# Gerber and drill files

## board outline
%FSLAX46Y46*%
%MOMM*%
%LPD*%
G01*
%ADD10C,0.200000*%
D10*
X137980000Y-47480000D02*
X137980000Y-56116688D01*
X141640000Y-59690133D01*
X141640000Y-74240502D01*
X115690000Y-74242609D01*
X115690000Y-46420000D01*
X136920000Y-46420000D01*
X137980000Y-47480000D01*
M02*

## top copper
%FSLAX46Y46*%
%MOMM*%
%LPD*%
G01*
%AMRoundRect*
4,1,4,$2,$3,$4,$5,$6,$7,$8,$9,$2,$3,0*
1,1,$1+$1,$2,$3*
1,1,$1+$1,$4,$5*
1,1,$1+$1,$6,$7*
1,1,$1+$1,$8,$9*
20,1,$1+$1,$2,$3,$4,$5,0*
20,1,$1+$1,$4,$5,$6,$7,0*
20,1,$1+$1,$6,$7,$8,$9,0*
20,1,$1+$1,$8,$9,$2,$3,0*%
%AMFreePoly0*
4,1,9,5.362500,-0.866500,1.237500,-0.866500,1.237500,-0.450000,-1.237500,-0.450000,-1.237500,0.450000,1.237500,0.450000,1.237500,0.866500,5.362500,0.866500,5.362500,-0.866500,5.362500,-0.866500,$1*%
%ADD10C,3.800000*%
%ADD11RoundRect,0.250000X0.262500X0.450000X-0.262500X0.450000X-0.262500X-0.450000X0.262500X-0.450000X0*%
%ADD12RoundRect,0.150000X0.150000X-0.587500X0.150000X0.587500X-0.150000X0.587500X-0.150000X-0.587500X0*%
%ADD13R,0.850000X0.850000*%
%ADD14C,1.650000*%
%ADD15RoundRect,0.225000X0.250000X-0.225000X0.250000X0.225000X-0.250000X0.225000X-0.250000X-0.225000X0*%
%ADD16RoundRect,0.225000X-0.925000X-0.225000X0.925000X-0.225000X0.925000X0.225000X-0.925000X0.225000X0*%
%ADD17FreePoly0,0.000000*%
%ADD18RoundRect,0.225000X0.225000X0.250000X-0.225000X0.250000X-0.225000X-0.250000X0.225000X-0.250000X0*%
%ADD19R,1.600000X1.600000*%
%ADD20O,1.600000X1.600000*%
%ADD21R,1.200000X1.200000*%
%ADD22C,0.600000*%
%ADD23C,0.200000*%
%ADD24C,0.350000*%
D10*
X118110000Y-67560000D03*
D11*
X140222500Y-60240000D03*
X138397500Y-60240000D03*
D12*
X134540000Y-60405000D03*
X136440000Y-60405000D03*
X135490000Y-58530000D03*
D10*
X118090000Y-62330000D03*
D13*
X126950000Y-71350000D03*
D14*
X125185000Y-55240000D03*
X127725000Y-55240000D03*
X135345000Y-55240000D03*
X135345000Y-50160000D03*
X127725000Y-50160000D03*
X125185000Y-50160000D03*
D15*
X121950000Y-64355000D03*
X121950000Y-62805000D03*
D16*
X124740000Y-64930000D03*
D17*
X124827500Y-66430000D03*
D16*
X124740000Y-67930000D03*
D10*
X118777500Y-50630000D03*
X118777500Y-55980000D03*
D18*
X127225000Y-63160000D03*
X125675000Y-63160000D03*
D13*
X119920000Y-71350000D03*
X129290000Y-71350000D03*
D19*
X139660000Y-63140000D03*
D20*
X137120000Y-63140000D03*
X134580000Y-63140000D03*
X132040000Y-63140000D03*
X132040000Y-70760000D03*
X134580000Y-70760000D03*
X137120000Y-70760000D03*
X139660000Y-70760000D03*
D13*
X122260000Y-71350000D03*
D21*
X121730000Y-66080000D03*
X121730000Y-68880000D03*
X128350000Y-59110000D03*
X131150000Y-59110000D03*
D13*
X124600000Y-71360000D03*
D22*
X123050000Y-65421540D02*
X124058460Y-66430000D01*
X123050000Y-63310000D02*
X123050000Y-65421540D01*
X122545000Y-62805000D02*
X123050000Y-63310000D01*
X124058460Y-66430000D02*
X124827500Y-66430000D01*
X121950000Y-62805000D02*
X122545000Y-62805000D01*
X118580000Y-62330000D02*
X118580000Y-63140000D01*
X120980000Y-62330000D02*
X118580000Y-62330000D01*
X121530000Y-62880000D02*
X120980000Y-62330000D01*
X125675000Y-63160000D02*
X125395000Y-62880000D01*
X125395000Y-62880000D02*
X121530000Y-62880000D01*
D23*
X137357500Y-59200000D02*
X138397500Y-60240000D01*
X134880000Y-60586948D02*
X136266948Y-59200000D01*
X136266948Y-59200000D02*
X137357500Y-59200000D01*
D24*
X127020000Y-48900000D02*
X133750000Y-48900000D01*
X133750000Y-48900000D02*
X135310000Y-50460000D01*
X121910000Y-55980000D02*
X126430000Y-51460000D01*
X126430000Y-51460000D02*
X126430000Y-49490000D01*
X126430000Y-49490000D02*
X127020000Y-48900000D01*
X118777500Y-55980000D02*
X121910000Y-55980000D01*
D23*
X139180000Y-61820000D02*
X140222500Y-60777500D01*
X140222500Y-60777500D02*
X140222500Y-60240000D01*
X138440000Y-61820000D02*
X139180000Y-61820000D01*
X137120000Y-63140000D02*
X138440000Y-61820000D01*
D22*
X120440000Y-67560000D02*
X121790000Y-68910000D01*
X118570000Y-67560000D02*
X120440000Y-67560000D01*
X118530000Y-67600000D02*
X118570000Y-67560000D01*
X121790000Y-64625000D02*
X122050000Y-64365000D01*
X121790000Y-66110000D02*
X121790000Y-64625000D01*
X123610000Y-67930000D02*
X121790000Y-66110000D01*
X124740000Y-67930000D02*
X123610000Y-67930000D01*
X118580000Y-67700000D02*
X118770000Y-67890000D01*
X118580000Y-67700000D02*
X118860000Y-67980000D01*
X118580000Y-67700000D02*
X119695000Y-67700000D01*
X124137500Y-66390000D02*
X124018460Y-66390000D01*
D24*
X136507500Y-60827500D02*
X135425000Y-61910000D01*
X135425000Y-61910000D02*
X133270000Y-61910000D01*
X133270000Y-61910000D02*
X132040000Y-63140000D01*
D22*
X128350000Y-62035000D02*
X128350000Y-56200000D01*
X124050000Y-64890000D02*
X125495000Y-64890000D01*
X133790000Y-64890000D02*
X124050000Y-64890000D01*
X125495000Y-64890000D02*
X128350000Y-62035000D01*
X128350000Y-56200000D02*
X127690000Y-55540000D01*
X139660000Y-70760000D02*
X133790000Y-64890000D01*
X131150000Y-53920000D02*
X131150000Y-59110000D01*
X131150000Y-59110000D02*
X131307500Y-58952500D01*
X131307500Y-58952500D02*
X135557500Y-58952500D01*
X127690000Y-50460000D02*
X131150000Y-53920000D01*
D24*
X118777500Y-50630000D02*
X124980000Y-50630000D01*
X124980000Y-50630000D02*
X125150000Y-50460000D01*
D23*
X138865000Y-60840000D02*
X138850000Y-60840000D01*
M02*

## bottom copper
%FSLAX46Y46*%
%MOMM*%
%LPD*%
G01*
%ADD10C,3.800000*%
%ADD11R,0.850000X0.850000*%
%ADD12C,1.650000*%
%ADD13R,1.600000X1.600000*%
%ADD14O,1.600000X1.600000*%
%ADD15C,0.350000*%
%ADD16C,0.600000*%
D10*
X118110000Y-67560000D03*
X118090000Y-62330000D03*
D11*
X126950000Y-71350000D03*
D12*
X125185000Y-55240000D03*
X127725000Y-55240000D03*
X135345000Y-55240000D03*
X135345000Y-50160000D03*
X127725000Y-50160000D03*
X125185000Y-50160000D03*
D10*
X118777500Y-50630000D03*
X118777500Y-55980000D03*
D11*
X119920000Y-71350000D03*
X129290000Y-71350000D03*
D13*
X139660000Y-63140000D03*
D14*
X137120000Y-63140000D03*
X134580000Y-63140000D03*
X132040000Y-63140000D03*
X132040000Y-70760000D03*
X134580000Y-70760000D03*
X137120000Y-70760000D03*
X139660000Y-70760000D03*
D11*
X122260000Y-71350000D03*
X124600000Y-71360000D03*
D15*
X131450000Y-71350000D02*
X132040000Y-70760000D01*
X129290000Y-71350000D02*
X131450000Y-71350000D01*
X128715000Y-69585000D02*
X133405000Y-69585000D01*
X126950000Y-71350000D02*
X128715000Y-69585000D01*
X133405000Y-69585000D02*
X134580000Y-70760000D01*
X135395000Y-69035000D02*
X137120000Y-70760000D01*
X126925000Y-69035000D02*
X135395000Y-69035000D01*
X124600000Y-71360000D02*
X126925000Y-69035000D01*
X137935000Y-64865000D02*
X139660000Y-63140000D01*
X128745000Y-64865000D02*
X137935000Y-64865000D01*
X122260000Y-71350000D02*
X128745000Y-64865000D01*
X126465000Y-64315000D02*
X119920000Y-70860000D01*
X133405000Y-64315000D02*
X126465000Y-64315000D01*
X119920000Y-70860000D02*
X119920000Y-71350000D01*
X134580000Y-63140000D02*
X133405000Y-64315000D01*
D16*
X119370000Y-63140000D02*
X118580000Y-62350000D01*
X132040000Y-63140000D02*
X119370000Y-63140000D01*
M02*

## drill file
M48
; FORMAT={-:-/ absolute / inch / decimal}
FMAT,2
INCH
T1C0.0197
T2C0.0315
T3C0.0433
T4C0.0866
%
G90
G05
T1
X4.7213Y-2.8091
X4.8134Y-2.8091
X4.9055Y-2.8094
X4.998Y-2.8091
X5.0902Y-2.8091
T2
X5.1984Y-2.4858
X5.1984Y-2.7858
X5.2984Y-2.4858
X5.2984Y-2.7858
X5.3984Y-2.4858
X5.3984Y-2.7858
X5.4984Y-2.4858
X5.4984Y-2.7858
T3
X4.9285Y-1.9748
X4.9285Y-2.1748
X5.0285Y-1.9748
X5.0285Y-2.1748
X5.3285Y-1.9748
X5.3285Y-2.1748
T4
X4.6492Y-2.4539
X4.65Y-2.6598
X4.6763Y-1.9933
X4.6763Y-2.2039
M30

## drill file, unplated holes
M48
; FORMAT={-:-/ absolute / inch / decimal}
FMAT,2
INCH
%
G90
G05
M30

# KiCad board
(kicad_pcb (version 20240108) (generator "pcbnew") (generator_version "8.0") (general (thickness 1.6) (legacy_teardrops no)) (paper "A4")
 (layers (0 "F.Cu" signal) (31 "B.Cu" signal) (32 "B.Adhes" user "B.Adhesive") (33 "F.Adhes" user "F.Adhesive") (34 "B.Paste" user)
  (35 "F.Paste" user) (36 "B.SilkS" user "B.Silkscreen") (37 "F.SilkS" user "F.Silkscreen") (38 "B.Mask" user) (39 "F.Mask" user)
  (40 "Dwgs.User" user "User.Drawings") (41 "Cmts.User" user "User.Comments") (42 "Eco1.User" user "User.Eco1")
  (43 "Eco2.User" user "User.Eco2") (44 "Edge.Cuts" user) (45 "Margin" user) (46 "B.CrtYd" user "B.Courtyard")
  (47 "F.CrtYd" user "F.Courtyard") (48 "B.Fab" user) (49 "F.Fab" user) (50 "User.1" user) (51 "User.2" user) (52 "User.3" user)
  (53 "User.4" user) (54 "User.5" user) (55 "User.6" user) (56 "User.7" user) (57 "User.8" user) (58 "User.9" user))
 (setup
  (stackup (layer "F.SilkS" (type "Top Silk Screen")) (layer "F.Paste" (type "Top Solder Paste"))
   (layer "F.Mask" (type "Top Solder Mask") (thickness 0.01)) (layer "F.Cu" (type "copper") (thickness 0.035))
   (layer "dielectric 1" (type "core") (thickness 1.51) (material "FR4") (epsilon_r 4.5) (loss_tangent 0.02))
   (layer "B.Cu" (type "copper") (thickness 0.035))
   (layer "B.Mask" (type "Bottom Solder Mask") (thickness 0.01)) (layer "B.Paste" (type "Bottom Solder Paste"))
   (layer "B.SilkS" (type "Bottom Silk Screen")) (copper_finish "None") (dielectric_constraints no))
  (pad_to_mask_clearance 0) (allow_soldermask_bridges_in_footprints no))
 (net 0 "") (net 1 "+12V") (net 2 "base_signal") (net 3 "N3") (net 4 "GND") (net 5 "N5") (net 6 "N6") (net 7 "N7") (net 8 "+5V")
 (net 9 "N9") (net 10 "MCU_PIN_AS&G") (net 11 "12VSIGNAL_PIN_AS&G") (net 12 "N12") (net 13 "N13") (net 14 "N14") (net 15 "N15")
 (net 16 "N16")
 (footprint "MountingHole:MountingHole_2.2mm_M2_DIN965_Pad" (layer "F.Cu") (at 118.11 67.56)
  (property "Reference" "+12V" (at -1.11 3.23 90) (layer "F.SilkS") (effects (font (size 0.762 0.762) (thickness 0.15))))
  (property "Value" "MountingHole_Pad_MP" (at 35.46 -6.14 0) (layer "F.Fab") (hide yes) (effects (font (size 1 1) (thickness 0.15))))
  (pad "1" thru_hole circle (at 0 0) (size 3.8 3.8) (drill 2.2) (layers "*.Cu" "*.Mask") (remove_unused_layers no) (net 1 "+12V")))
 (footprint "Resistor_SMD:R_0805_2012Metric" (layer "F.Cu") (at 139.31 60.24 180)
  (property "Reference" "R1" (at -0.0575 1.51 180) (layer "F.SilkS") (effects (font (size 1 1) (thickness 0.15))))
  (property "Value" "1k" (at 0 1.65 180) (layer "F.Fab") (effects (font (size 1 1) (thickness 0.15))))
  (pad "1" smd roundrect (at -0.9125 0 180) (size 1.025 1.4) (layers "F.Cu" "F.Paste" "F.Mask") (roundrect_rratio 0.243902)
   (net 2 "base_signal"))
  (pad "2" smd roundrect (at 0.9125 0 180) (size 1.025 1.4) (layers "F.Cu" "F.Paste" "F.Mask") (roundrect_rratio 0.243902) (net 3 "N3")))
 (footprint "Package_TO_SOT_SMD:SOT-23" (layer "F.Cu") (at 135.49 59.4675 90)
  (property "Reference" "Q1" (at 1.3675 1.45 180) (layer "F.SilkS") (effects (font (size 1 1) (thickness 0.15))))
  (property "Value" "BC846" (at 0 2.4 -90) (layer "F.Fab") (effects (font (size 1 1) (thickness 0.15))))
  (pad "1" smd roundrect (at -0.9375 -0.95 90) (size 1.475 0.6) (layers "F.Cu" "F.Paste" "F.Mask") (roundrect_rratio 0.25) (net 3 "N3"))
  (pad "2" smd roundrect (at -0.9375 0.95 90) (size 1.475 0.6) (layers "F.Cu" "F.Paste" "F.Mask") (roundrect_rratio 0.25) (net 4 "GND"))
  (pad "3" smd roundrect (at 0.9375 0 90) (size 1.475 0.6) (layers "F.Cu" "F.Paste" "F.Mask") (roundrect_rratio 0.25) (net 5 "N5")))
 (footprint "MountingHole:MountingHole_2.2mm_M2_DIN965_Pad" (layer "F.Cu") (at 118.09 62.33)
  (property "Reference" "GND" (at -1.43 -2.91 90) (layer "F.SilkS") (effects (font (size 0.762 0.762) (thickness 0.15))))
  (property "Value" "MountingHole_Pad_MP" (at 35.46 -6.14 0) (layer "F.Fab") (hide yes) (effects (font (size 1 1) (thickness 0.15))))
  (pad "1" thru_hole circle (at 0 0) (size 3.8 3.8) (drill 2.2) (layers "*.Cu" "*.Mask") (remove_unused_layers no) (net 4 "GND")))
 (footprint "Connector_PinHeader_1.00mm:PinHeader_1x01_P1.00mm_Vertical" (layer "F.Cu") (at 126.95 71.35)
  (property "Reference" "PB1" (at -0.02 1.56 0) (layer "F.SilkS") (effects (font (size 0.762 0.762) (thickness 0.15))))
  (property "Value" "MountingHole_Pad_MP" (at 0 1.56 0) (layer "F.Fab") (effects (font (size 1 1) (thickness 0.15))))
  (pad "1" thru_hole rect (at 0 0) (size 0.85 0.85) (drill 0.5) (layers "*.Cu" "*.Mask") (remove_unused_layers no) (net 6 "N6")))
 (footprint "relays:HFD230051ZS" (layer "F.Cu") (at 125.185 55.24)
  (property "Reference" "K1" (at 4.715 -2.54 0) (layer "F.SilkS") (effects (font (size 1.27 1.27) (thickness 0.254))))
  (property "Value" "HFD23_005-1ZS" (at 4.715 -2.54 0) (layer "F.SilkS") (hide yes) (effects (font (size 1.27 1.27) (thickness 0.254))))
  (pad "1" thru_hole circle (at 0 0) (size 1.65 1.65) (drill 1.1) (layers "*.Cu" "*.Mask") (remove_unused_layers no) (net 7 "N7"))
  (pad "2" thru_hole circle (at 2.54 0) (size 1.65 1.65) (drill 1.1) (layers "*.Cu" "*.Mask") (remove_unused_layers no) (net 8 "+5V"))
  (pad "3" thru_hole circle (at 10.16 0) (size 1.65 1.65) (drill 1.1) (layers "*.Cu" "*.Mask") (remove_unused_layers no) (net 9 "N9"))
  (pad "4" thru_hole circle (at 10.16 -5.08) (size 1.65 1.65) (drill 1.1) (layers "*.Cu" "*.Mask") (remove_unused_layers no)
   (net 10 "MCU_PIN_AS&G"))
  (pad "5" thru_hole circle (at 2.54 -5.08) (size 1.65 1.65) (drill 1.1) (layers "*.Cu" "*.Mask") (remove_unused_layers no) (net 5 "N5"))
  (pad "6" thru_hole circle (at 0 -5.08) (size 1.65 1.65) (drill 1.1) (layers "*.Cu" "*.Mask") (remove_unused_layers no)
   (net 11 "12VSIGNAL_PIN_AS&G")))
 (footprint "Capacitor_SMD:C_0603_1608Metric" (layer "F.Cu") (at 121.95 63.58 90)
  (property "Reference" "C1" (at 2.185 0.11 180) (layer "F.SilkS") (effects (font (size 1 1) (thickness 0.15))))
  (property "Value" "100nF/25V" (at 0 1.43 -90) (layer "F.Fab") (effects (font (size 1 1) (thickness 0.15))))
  (pad "1" smd roundrect (at -0.775 0 90) (size 0.9 0.95) (layers "F.Cu" "F.Paste" "F.Mask") (roundrect_rratio 0.25) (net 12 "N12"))
  (pad "2" smd roundrect (at 0.775 0 90) (size 0.9 0.95) (layers "F.Cu" "F.Paste" "F.Mask") (roundrect_rratio 0.25) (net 4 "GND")))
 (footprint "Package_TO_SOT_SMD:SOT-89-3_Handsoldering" (layer "F.Cu") (at 127.19 66.43)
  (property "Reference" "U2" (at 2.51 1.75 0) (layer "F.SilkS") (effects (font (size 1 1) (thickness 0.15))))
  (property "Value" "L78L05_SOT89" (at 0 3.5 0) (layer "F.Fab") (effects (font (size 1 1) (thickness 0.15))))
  (pad "1" smd roundrect (at -2.45 -1.5) (size 2.3 0.9) (layers "F.Cu" "F.Paste" "F.Mask") (roundrect_rratio 0.25) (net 8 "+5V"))
  (pad "2" smd custom (at -2.3625 0) (size 2.475 0.9) (layers "F.Cu" "F.Paste" "F.Mask") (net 4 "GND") (zone_connect 2)
   (thermal_bridge_angle 45) (options (clearance outline) (anchor rect)) (primitives))
  (pad "3" smd roundrect (at -2.45 1.5) (size 2.3 0.9) (layers "F.Cu" "F.Paste" "F.Mask") (roundrect_rratio 0.25) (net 12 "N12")))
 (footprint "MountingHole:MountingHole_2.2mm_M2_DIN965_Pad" (layer "F.Cu") (at 118.7775 50.63)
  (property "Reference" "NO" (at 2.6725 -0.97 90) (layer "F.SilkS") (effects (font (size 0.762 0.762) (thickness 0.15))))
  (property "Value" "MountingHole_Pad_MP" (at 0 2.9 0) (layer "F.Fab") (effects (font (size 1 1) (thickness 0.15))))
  (pad "1" thru_hole circle (at 0 0) (size 3.8 3.8) (drill 2.2) (layers "*.Cu" "*.Mask") (remove_unused_layers no)
   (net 11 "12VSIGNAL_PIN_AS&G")))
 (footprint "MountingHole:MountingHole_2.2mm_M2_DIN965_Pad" (layer "F.Cu") (at 118.7775 55.98)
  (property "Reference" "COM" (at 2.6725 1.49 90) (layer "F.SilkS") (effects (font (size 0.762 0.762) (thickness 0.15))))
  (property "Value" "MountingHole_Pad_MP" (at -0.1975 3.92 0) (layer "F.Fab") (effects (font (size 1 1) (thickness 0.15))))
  (pad "1" thru_hole circle (at 0 0) (size 3.8 3.8) (drill 2.2) (layers "*.Cu" "*.Mask") (remove_unused_layers no) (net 10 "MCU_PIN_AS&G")))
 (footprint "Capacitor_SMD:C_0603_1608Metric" (layer "F.Cu") (at 126.45 63.16 180)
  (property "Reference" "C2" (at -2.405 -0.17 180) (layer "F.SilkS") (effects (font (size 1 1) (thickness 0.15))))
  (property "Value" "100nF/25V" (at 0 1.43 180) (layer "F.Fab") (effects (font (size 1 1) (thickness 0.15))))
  (pad "1" smd roundrect (at -0.775 0 180) (size 0.9 0.95) (layers "F.Cu" "F.Paste" "F.Mask") (roundrect_rratio 0.25) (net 8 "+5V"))
  (pad "2" smd roundrect (at 0.775 0 180) (size 0.9 0.95) (layers "F.Cu" "F.Paste" "F.Mask") (roundrect_rratio 0.25) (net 4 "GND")))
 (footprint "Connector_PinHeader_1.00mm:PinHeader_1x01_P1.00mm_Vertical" (layer "F.Cu") (at 119.92 71.35)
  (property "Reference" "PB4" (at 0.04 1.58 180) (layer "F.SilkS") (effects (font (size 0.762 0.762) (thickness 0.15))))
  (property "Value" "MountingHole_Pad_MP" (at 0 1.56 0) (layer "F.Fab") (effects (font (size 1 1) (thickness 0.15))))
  (pad "1" thru_hole rect (at 0 0) (size 0.85 0.85) (drill 0.5) (layers "*.Cu" "*.Mask") (remove_unused_layers no) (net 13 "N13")))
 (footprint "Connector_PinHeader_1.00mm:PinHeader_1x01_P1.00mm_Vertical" (layer "F.Cu") (at 129.29 71.35)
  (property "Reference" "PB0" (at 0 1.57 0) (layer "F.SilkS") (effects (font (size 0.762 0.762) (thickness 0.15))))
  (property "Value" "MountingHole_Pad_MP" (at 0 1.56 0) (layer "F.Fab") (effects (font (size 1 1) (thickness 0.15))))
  (pad "1" thru_hole rect (at 0 0) (size 0.85 0.85) (drill 0.5) (layers "*.Cu" "*.Mask") (remove_unused_layers no) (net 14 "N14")))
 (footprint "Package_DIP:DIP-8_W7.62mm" (layer "F.Cu") (at 139.66 63.14 -90)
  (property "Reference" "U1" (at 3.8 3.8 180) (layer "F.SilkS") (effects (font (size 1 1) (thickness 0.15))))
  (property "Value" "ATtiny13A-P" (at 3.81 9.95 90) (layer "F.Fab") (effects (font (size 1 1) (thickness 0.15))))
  (pad "1" thru_hole rect (at 0 0 270) (size 1.6 1.6) (drill 0.8) (layers "*.Cu" "*.Mask") (remove_unused_layers no) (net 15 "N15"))
  (pad "2" thru_hole oval (at 0 2.54 270) (size 1.6 1.6) (drill 0.8) (layers "*.Cu" "*.Mask") (remove_unused_layers no)
   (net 2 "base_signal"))
  (pad "3" thru_hole oval (at 0 5.08 270) (size 1.6 1.6) (drill 0.8) (layers "*.Cu" "*.Mask") (remove_unused_layers no) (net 13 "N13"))
  (pad "4" thru_hole oval (at 0 7.62 270) (size 1.6 1.6) (drill 0.8) (layers "*.Cu" "*.Mask") (remove_unused_layers no) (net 4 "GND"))
  (pad "5" thru_hole oval (at 7.62 7.62 270) (size 1.6 1.6) (drill 0.8) (layers "*.Cu" "*.Mask") (remove_unused_layers no) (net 14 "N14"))
  (pad "6" thru_hole oval (at 7.62 5.08 270) (size 1.6 1.6) (drill 0.8) (layers "*.Cu" "*.Mask") (remove_unused_layers no) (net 6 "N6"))
  (pad "7" thru_hole oval (at 7.62 2.54 270) (size 1.6 1.6) (drill 0.8) (layers "*.Cu" "*.Mask") (remove_unused_layers no) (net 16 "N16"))
  (pad "8" thru_hole oval (at 7.62 0 270) (size 1.6 1.6) (drill 0.8) (layers "*.Cu" "*.Mask") (remove_unused_layers no) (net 8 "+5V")))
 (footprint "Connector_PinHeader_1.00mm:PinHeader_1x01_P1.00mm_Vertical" (layer "F.Cu") (at 122.26 71.35)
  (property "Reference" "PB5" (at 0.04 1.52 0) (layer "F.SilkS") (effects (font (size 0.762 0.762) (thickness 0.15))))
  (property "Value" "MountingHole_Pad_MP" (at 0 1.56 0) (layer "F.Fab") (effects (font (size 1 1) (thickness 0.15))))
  (pad "1" thru_hole rect (at 0 0) (size 0.85 0.85) (drill 0.5) (layers "*.Cu" "*.Mask") (remove_unused_layers no) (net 15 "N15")))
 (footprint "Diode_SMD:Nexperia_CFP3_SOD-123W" (layer "F.Cu") (at 121.73 67.48 -90)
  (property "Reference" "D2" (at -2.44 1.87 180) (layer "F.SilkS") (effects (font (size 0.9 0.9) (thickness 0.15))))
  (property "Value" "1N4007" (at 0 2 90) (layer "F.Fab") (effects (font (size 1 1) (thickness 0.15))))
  (pad "1" smd rect (at -1.4 0 270) (size 1.2 1.2) (layers "F.Cu" "F.Paste" "F.Mask") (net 12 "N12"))
  (pad "2" smd rect (at 1.4 0 270) (size 1.2 1.2) (layers "F.Cu" "F.Paste" "F.Mask") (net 1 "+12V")))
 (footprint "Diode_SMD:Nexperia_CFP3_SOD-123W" (layer "F.Cu") (at 129.75 59.11)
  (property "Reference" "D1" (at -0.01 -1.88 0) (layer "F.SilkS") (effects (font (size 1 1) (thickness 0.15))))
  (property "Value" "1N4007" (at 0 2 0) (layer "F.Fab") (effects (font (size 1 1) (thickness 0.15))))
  (pad "1" smd rect (at -1.4 0) (size 1.2 1.2) (layers "F.Cu" "F.Paste" "F.Mask") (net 8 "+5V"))
  (pad "2" smd rect (at 1.4 0) (size 1.2 1.2) (layers "F.Cu" "F.Paste" "F.Mask") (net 5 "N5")))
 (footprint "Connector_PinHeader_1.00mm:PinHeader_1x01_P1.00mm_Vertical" (layer "F.Cu") (at 124.6 71.36)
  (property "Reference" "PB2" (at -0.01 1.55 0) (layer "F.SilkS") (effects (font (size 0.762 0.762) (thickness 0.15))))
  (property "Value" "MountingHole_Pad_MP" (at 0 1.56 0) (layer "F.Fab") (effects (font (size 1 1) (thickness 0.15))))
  (pad "1" thru_hole rect (at 0 0) (size 0.85 0.85) (drill 0.5) (layers "*.Cu" "*.Mask") (remove_unused_layers no) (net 16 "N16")))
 (gr_poly
  (pts (xy 115.69 74.242609) (xy 141.64 74.240502) (xy 141.64 59.690133) (xy 137.98 56.116688) (xy 137.98 47.48) (xy 136.92 46.42)
   (xy 115.69 46.42))
  (stroke (width 0.2) (type solid)) (fill none) (layer "Edge.Cuts"))
 (segment (start 118.58 67.7) (end 118.77 67.89) (width 0.6) (layer "F.Cu") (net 1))
 (segment (start 118.57 67.56) (end 120.44 67.56) (width 0.6) (layer "F.Cu") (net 1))
 (segment (start 118.53 67.6) (end 118.57 67.56) (width 0.6) (layer "F.Cu") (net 1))
 (segment (start 120.44 67.56) (end 121.79 68.91) (width 0.6) (layer "F.Cu") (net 1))
 (segment (start 118.58 67.7) (end 118.86 67.98) (width 0.6) (layer "F.Cu") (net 1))
 (segment (start 118.58 67.7) (end 119.695 67.7) (width 0.6) (layer "F.Cu") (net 1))
 (segment (start 125.395 62.88) (end 121.53 62.88) (width 0.6) (layer "F.Cu") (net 4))
 (segment (start 124.1375 66.39) (end 124.01846 66.39) (width 0.6) (layer "F.Cu") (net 4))
 (segment (start 121.53 62.88) (end 120.98 62.33) (width 0.6) (layer "F.Cu") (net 4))
 (segment (start 125.675 63.16) (end 125.395 62.88) (width 0.6) (layer "F.Cu") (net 4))
 (segment (start 136.5075 60.8275) (end 135.425 61.91) (width 0.35) (layer "F.Cu") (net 4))
 (segment (start 123.05 63.31) (end 123.05 65.42154) (width 0.6) (layer "F.Cu") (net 4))
 (segment (start 123.05 65.42154) (end 124.05846 66.43) (width 0.6) (layer "F.Cu") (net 4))
 (segment (start 120.98 62.33) (end 118.58 62.33) (width 0.6) (layer "F.Cu") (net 4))
 (segment (start 135.425 61.91) (end 133.27 61.91) (width 0.35) (layer "F.Cu") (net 4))
 (segment (start 122.545 62.805) (end 123.05 63.31) (width 0.6) (layer "F.Cu") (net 4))
 (segment (start 118.58 62.33) (end 118.58 63.14) (width 0.6) (layer "F.Cu") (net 4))
 (segment (start 121.95 62.805) (end 122.545 62.805) (width 0.6) (layer "F.Cu") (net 4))
 (segment (start 124.05846 66.43) (end 124.8275 66.43) (width 0.6) (layer "F.Cu") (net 4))
 (segment (start 133.27 61.91) (end 132.04 63.14) (width 0.35) (layer "F.Cu") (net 4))
 (segment (start 119.37 63.14) (end 118.58 62.35) (width 0.6) (layer "B.Cu") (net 4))
 (segment (start 132.04 63.14) (end 119.37 63.14) (width 0.6) (layer "B.Cu") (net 4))
 (segment (start 128.35 62.035) (end 128.35 56.2) (width 0.6) (layer "F.Cu") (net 8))
 (segment (start 124.05 64.89) (end 125.495 64.89) (width 0.6) (layer "F.Cu") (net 8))
 (segment (start 133.79 64.89) (end 124.05 64.89) (width 0.6) (layer "F.Cu") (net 8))
 (segment (start 125.495 64.89) (end 128.35 62.035) (width 0.6) (layer "F.Cu") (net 8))
 (segment (start 128.35 56.2) (end 127.69 55.54) (width 0.6) (layer "F.Cu") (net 8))
 (segment (start 139.66 70.76) (end 133.79 64.89) (width 0.6) (layer "F.Cu") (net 8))
 (segment (start 131.15 53.92) (end 131.15 59.11) (width 0.6) (layer "F.Cu") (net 5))
 (segment (start 131.15 59.11) (end 131.3075 58.9525) (width 0.6) (layer "F.Cu") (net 5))
 (segment (start 131.3075 58.9525) (end 135.5575 58.9525) (width 0.6) (layer "F.Cu") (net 5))
 (segment (start 127.69 50.46) (end 131.15 53.92) (width 0.6) (layer "F.Cu") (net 5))
 (segment (start 118.7775 50.63) (end 124.98 50.63) (width 0.35) (layer "F.Cu") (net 11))
 (segment (start 124.98 50.63) (end 125.15 50.46) (width 0.35) (layer "F.Cu") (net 11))
 (segment (start 127.02 48.9) (end 133.75 48.9) (width 0.35) (layer "F.Cu") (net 10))
 (segment (start 118.7775 55.98) (end 121.91 55.98) (width 0.35) (layer "F.Cu") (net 10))
 (segment (start 121.91 55.98) (end 126.43 51.46) (width 0.35) (layer "F.Cu") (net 10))
 (segment (start 126.43 51.46) (end 126.43 49.49) (width 0.35) (layer "F.Cu") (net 10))
 (segment (start 126.43 49.49) (end 127.02 48.9) (width 0.35) (layer "F.Cu") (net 10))
 (segment (start 133.75 48.9) (end 135.31 50.46) (width 0.35) (layer "F.Cu") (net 10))
 (segment (start 131.45 71.35) (end 132.04 70.76) (width 0.35) (layer "B.Cu") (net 14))
 (segment (start 129.29 71.35) (end 131.45 71.35) (width 0.35) (layer "B.Cu") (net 14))
 (segment (start 126.95 71.35) (end 128.715 69.585) (width 0.35) (layer "B.Cu") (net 6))
 (segment (start 133.405 69.585) (end 134.58 70.76) (width 0.35) (layer "B.Cu") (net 6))
 (segment (start 128.715 69.585) (end 133.405 69.585) (width 0.35) (layer "B.Cu") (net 6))
 (segment (start 126.925 69.035) (end 135.395 69.035) (width 0.35) (layer "B.Cu") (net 16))
 (segment (start 135.395 69.035) (end 137.12 70.76) (width 0.35) (layer "B.Cu") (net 16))
 (segment (start 124.6 71.36) (end 126.925 69.035) (width 0.35) (layer "B.Cu") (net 16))
 (segment (start 119.92 70.86) (end 119.92 71.35) (width 0.35) (layer "B.Cu") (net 13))
 (segment (start 134.58 63.14) (end 133.405 64.315) (width 0.35) (layer "B.Cu") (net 13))
 (segment (start 126.465 64.315) (end 119.92 70.86) (width 0.35) (layer "B.Cu") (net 13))
 (segment (start 133.405 64.315) (end 126.465 64.315) (width 0.35) (layer "B.Cu") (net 13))
 (segment (start 137.935 64.865) (end 139.66 63.14) (width 0.35) (layer "B.Cu") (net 15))
 (segment (start 128.745 64.865) (end 137.935 64.865) (width 0.35) (layer "B.Cu") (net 15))
 (segment (start 122.26 71.35) (end 128.745 64.865) (width 0.35) (layer "B.Cu") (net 15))
 (segment (start 136.266948 59.2) (end 137.3575 59.2) (width 0.2) (layer "F.Cu") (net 3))
 (segment (start 134.88 60.586948) (end 136.266948 59.2) (width 0.2) (layer "F.Cu") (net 3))
 (segment (start 137.3575 59.2) (end 138.3975 60.24) (width 0.2) (layer "F.Cu") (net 3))
 (segment (start 138.865 60.84) (end 138.85 60.84) (width 0.2) (layer "F.Cu") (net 3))
 (segment (start 137.12 63.14) (end 138.44 61.82) (width 0.2) (layer "F.Cu") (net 2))
 (segment (start 140.2225 60.7775) (end 140.2225 60.24) (width 0.2) (layer "F.Cu") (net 2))
 (segment (start 138.44 61.82) (end 139.18 61.82) (width 0.2) (layer "F.Cu") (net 2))
 (segment (start 139.18 61.82) (end 140.2225 60.7775) (width 0.2) (layer "F.Cu") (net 2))
 (segment (start 121.79 64.625) (end 122.05 64.365) (width 0.6) (layer "F.Cu") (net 12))
 (segment (start 124.74 67.93) (end 123.61 67.93) (width 0.6) (layer "F.Cu") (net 12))
 (segment (start 121.79 66.11) (end 121.79 64.625) (width 0.6) (layer "F.Cu") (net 12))
 (segment (start 123.61 67.93) (end 121.79 66.11) (width 0.6) (layer "F.Cu") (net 12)))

